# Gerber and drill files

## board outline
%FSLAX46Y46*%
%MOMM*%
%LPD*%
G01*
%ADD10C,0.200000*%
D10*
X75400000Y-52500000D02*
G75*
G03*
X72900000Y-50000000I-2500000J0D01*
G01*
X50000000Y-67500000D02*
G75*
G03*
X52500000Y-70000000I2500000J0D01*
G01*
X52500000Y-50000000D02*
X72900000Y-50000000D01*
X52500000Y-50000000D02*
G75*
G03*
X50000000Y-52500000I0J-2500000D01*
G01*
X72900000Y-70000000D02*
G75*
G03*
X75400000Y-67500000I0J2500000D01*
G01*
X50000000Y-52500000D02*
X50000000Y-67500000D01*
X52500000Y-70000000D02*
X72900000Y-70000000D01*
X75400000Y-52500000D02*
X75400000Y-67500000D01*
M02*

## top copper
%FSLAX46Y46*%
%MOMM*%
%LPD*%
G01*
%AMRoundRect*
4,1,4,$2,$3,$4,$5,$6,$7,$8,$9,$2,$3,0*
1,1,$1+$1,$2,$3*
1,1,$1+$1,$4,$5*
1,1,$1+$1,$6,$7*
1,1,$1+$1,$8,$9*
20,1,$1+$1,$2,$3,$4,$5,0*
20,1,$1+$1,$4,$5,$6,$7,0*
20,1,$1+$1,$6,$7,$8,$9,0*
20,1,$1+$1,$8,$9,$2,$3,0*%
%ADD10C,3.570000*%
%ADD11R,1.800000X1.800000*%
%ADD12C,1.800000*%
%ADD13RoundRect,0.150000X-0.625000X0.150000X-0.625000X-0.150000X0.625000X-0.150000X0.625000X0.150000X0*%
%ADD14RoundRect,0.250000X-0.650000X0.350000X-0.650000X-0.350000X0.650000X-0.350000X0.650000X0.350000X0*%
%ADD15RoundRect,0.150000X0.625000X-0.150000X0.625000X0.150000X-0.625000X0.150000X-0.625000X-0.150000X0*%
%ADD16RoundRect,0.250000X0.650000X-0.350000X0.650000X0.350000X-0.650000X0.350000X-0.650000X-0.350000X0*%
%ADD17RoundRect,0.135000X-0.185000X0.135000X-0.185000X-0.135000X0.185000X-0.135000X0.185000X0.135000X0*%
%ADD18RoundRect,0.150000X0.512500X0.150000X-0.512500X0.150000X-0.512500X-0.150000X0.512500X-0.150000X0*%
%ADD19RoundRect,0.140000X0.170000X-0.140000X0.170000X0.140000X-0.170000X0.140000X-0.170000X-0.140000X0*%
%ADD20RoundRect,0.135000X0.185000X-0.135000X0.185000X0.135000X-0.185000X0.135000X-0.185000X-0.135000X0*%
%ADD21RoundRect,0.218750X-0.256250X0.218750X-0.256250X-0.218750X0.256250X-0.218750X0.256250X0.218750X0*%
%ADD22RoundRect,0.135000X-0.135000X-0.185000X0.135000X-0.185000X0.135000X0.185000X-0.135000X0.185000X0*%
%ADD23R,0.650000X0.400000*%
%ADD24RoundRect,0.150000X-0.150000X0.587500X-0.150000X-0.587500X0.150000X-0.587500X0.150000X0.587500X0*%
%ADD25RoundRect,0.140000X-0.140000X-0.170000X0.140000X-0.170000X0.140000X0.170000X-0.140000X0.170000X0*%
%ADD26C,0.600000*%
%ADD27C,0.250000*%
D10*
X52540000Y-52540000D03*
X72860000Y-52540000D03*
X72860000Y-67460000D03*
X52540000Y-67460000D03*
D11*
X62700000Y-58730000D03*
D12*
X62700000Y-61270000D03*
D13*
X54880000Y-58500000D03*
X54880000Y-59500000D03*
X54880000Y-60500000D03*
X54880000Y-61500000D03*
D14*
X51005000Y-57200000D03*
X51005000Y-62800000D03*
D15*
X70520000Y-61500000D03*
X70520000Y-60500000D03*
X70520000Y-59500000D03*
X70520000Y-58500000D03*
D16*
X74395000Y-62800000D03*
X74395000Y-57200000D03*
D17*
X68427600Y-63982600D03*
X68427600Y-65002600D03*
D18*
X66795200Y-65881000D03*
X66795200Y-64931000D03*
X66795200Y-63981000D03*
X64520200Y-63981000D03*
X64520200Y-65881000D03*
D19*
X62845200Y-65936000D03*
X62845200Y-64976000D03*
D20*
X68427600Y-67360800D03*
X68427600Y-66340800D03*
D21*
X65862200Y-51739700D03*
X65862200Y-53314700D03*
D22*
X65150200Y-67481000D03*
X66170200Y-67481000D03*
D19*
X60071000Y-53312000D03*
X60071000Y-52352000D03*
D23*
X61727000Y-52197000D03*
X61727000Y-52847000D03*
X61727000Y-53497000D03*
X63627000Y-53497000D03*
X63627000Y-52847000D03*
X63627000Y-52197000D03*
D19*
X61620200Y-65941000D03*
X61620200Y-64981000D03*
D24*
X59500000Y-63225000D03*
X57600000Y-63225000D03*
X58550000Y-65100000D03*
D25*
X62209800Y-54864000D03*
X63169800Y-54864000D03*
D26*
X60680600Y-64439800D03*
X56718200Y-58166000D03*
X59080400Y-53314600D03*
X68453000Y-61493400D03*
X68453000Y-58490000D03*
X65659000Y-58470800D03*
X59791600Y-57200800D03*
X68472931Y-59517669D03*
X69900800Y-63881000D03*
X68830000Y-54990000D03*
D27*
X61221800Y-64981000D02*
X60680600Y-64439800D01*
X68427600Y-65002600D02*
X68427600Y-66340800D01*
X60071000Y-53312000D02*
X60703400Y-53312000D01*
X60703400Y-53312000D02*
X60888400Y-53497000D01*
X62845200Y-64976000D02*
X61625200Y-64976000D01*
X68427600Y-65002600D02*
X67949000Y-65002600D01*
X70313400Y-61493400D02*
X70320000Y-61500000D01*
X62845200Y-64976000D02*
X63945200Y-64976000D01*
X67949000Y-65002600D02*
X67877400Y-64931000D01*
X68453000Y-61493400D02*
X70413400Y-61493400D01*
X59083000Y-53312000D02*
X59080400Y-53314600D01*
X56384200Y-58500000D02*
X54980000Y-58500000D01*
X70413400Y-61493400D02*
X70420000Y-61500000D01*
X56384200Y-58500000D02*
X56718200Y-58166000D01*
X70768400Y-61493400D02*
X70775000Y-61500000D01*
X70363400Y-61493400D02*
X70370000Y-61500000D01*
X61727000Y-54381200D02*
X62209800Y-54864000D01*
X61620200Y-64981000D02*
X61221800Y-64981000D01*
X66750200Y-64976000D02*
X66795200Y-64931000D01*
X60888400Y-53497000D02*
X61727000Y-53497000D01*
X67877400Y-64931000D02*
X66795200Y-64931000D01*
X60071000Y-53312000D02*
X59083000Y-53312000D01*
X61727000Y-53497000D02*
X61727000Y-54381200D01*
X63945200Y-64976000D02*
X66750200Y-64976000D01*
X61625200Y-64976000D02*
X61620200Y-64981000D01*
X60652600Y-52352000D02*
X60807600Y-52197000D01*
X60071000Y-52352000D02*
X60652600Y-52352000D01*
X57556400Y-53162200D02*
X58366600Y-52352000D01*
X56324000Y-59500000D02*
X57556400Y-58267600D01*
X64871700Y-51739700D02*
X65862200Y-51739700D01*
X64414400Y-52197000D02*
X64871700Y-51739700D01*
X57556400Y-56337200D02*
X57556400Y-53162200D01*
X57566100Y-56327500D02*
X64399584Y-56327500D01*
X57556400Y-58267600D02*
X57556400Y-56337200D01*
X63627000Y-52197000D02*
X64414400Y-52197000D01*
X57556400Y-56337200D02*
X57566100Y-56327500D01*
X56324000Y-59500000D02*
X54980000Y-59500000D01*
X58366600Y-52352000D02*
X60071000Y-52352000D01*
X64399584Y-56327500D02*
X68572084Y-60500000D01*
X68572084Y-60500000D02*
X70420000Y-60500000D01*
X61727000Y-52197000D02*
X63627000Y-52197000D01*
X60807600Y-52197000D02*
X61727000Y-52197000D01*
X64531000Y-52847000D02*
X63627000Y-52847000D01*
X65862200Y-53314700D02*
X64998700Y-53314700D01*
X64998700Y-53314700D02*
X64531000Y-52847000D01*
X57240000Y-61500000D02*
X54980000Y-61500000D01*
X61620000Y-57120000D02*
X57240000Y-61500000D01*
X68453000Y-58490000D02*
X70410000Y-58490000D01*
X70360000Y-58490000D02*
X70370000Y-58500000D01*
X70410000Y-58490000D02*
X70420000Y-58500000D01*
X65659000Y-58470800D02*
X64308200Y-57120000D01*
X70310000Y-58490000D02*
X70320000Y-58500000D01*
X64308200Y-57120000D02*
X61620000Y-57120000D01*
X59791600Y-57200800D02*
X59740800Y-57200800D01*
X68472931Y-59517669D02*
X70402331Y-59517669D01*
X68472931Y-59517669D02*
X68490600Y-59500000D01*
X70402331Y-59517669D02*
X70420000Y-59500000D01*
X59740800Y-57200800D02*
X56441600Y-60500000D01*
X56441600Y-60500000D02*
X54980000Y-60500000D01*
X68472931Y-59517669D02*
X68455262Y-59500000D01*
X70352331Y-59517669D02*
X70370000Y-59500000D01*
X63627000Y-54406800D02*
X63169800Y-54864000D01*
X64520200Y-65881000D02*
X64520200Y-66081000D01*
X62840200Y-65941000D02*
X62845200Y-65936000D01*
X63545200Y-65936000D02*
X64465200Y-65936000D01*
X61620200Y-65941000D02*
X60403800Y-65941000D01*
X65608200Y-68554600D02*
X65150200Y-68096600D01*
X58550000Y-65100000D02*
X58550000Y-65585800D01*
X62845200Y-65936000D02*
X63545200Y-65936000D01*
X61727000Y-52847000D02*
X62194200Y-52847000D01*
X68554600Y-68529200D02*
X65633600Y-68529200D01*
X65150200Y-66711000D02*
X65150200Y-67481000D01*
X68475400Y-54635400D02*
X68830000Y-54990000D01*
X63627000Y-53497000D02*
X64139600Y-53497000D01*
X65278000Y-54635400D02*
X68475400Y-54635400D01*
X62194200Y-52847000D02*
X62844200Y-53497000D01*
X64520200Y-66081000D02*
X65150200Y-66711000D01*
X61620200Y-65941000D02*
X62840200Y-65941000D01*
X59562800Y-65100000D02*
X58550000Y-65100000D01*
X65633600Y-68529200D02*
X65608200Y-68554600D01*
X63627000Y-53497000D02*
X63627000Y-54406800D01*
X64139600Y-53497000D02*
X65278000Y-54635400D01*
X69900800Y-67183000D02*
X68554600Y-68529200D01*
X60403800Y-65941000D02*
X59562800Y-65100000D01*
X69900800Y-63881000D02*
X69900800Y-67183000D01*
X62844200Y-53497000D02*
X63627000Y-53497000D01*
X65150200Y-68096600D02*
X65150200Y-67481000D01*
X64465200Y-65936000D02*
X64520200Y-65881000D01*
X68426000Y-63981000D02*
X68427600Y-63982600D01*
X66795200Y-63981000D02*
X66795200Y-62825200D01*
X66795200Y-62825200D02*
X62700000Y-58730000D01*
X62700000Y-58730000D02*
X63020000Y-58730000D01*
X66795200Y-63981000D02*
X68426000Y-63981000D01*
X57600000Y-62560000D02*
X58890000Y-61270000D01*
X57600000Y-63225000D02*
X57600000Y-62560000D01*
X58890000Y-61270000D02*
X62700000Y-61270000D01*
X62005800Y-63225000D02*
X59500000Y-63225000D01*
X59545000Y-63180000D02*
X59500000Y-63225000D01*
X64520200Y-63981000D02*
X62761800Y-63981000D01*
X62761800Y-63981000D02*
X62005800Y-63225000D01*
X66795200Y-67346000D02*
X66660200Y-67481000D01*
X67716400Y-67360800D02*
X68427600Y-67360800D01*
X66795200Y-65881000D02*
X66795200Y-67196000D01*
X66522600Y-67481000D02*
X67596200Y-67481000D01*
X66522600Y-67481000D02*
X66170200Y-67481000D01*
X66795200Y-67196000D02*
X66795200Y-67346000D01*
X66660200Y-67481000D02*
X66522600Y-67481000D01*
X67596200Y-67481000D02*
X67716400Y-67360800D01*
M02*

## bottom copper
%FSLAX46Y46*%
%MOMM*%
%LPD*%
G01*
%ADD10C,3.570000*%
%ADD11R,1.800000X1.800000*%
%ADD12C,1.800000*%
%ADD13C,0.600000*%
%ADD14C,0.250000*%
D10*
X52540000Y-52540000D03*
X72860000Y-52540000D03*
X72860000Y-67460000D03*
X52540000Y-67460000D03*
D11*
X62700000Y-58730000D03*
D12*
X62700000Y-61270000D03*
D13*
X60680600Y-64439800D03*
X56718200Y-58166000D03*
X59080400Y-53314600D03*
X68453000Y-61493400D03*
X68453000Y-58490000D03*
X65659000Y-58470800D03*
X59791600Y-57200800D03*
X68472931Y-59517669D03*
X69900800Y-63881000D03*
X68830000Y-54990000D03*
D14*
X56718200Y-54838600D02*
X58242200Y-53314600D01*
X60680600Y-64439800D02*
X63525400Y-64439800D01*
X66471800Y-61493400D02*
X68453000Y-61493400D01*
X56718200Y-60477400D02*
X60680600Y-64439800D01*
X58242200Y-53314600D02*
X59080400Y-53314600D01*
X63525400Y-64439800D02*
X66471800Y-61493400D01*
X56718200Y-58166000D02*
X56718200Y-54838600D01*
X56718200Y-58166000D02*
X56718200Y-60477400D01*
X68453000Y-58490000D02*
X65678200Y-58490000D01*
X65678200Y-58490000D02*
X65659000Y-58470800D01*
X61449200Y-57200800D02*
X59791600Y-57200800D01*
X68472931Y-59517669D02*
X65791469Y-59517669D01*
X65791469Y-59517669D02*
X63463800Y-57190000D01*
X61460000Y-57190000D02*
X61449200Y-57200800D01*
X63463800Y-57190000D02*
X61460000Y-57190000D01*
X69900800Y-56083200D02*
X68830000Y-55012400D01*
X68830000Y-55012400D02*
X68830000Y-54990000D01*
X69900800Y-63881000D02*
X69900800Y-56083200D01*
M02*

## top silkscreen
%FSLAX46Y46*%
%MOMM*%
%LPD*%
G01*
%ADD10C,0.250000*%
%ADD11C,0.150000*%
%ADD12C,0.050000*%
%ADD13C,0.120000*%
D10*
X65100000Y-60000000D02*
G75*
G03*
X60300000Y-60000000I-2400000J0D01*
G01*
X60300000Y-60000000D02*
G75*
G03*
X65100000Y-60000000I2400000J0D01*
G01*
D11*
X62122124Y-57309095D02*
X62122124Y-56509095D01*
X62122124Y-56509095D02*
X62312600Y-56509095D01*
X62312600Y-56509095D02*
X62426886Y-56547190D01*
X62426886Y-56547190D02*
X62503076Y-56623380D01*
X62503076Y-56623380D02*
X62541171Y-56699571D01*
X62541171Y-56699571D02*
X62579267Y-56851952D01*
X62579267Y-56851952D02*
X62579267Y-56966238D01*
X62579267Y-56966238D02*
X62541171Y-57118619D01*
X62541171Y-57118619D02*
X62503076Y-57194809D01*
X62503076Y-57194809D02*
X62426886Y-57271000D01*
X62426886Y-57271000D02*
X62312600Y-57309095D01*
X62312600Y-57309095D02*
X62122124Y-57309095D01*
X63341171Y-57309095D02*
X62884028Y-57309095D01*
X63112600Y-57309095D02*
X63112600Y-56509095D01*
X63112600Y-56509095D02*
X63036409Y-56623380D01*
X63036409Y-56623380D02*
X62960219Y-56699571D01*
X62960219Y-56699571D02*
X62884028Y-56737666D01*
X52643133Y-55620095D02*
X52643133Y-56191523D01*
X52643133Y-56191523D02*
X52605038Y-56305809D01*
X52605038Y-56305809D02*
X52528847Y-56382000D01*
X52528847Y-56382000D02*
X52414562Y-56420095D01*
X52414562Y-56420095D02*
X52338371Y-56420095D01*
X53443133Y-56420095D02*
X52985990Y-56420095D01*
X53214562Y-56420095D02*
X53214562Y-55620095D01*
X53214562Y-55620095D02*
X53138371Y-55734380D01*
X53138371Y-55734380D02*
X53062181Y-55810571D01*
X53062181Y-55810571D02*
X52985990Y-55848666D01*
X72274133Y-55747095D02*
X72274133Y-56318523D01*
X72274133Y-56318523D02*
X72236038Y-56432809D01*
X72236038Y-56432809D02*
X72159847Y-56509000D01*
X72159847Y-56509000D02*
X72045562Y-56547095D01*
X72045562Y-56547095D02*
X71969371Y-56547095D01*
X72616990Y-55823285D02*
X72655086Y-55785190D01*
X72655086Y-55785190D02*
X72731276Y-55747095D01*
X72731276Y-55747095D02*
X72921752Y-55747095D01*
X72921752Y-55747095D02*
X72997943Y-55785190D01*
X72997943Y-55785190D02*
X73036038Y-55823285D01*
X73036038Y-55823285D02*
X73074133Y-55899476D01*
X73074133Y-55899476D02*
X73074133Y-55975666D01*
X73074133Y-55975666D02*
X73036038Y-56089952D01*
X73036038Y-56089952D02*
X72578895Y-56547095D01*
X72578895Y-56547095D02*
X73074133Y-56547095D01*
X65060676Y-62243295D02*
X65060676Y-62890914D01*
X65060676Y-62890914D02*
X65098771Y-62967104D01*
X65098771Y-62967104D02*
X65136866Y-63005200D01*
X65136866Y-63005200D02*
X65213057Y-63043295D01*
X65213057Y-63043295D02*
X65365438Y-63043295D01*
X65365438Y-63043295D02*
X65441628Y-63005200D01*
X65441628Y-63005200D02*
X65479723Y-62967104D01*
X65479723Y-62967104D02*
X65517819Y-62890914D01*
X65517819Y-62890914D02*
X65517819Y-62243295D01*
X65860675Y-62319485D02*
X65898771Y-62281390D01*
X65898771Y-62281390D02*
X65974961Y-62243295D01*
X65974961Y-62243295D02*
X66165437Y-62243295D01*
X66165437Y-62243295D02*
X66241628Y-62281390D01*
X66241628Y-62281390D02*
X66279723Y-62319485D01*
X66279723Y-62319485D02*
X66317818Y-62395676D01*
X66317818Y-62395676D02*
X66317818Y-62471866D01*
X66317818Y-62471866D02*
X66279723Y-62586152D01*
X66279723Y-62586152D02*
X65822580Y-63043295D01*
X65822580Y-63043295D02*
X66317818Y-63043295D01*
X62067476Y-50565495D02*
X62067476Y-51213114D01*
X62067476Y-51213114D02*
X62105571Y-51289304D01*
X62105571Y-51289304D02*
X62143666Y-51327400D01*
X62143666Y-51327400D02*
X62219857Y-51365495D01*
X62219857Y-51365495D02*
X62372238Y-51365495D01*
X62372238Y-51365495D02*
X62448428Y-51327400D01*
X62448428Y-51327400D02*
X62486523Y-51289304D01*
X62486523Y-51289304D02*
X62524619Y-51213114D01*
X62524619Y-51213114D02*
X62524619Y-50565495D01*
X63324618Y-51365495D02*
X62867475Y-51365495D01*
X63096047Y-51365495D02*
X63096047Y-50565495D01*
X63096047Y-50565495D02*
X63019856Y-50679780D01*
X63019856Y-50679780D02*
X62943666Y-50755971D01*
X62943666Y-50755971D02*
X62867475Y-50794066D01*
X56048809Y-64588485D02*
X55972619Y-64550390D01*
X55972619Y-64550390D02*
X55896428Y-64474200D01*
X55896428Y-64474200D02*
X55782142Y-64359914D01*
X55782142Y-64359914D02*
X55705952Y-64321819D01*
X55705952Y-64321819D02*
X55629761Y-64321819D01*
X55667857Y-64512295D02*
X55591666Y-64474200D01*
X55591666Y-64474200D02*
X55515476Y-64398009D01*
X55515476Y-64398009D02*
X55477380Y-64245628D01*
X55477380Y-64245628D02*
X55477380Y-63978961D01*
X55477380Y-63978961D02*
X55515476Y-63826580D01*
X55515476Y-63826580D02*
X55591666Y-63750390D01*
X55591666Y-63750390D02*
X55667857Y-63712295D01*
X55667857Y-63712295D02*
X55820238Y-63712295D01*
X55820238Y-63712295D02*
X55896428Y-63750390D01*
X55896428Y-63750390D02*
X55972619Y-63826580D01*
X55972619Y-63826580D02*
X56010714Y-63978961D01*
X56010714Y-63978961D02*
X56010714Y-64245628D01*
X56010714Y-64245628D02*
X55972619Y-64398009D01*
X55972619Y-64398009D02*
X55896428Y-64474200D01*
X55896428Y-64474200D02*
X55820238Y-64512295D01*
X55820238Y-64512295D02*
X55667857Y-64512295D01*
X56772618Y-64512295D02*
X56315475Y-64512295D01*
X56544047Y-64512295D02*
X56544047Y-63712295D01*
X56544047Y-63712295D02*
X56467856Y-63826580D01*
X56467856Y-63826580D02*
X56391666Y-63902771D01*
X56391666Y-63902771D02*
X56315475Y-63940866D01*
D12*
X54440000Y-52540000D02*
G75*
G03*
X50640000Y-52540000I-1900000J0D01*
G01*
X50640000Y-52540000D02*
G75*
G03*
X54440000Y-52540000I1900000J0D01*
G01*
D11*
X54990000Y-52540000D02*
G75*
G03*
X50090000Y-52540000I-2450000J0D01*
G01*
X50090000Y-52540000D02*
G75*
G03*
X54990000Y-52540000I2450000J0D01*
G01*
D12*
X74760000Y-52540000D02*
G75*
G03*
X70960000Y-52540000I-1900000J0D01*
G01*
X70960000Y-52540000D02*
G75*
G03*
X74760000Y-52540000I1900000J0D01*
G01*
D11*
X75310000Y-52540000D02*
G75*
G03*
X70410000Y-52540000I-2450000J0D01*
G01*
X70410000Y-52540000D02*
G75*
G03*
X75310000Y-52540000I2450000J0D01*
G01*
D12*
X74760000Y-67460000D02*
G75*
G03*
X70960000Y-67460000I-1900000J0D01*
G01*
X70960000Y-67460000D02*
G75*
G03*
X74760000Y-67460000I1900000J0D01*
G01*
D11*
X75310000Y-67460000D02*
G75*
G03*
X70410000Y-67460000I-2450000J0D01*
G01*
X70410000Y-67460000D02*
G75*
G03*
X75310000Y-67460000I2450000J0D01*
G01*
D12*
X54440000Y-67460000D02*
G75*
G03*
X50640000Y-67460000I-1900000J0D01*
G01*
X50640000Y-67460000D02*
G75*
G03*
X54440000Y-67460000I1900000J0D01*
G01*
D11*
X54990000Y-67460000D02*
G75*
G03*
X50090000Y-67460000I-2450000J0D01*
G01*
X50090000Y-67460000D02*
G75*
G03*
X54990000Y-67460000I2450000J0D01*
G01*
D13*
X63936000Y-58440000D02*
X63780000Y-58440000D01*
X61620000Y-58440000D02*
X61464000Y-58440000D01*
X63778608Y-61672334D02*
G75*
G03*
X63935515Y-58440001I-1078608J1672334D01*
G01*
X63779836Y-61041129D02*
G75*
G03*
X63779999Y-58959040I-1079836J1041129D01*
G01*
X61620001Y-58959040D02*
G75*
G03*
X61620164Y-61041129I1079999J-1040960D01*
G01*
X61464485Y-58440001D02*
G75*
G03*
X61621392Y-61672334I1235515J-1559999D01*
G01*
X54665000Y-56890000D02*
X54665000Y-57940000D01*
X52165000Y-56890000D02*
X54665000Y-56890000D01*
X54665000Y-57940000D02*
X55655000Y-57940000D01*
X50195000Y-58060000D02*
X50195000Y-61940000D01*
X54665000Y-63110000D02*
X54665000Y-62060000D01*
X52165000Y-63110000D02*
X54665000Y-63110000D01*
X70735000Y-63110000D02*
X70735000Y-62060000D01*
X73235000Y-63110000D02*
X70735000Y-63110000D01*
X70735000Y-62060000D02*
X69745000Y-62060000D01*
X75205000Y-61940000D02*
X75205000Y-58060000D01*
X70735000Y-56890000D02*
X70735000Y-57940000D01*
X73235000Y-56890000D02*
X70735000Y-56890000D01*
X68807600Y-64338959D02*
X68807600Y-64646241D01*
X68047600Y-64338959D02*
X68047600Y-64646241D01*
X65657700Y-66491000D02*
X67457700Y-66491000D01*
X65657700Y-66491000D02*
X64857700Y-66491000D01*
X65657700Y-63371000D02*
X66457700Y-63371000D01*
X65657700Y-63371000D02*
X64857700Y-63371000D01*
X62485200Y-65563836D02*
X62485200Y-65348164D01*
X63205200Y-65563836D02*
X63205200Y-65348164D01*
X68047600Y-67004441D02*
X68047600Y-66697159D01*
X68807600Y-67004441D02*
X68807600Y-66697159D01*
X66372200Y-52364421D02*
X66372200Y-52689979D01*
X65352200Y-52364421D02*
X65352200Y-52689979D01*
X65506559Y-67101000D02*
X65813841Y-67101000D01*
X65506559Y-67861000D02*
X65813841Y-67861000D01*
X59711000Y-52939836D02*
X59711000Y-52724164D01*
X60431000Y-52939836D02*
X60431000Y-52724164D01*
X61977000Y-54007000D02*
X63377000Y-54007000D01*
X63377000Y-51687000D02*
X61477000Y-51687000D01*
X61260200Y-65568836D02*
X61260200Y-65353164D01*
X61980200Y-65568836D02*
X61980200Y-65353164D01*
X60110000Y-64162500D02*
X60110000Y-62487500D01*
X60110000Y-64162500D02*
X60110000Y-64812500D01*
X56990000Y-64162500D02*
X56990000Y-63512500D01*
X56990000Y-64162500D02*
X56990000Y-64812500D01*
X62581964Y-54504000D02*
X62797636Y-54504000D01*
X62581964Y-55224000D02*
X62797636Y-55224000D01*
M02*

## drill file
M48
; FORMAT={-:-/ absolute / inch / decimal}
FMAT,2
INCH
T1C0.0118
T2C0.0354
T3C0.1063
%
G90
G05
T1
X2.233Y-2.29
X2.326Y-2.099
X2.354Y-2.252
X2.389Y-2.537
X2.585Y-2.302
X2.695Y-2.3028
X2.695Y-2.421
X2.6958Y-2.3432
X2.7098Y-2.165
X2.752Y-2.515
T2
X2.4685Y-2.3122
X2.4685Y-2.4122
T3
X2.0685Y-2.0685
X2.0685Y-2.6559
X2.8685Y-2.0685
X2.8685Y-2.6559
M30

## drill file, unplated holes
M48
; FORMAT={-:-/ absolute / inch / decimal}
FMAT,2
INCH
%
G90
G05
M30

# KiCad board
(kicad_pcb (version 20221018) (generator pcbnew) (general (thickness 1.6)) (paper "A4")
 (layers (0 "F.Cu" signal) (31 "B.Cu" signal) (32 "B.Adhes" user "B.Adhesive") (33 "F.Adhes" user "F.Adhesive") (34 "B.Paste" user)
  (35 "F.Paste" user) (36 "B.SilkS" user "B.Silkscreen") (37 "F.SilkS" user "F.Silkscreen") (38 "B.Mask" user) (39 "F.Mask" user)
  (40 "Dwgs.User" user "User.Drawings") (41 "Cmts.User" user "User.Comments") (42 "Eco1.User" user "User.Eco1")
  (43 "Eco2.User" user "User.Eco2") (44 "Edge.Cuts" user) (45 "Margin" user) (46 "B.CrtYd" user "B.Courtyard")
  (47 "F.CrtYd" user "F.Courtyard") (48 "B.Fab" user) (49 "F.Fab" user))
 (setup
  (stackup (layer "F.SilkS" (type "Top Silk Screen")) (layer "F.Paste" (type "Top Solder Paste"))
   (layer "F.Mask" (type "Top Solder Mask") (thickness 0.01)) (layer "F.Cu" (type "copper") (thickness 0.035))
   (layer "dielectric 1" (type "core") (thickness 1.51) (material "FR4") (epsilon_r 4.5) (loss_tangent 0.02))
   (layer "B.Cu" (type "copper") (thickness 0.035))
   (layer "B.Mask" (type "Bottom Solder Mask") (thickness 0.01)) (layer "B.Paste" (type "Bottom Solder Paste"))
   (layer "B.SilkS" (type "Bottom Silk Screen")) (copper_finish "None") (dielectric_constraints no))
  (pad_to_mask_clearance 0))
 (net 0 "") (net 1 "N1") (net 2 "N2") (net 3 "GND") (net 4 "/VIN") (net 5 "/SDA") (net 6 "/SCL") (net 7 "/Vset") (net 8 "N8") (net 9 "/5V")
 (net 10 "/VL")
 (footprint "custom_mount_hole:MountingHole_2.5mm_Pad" (layer "F.Cu") (at 52.54 52.54)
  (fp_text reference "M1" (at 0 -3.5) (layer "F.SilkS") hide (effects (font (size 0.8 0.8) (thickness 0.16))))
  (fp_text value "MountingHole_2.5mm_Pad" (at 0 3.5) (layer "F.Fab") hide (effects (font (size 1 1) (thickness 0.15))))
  (fp_circle (center 0 0) (end 1.9 0) (stroke (width 0.05) (type solid)) (fill none) (layer "F.SilkS"))
  (fp_circle (center 0 0) (end 2.45 0) (stroke (width 0.15) (type solid)) (fill none) (layer "F.SilkS"))
  (pad "~" thru_hole circle (at 0 0) (size 3.57 3.57) (drill 2.7) (layers "*.Cu" "*.Mask")))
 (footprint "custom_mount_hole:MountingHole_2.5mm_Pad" (layer "F.Cu") (at 72.86 52.54)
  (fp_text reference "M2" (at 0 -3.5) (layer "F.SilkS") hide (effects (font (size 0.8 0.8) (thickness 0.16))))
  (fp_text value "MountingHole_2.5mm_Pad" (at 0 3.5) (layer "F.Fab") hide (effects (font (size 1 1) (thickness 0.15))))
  (fp_circle (center 0 0) (end 1.9 0) (stroke (width 0.05) (type solid)) (fill none) (layer "F.SilkS"))
  (fp_circle (center 0 0) (end 2.45 0) (stroke (width 0.15) (type solid)) (fill none) (layer "F.SilkS"))
  (pad "~" thru_hole circle (at 0 0) (size 3.57 3.57) (drill 2.7) (layers "*.Cu" "*.Mask")))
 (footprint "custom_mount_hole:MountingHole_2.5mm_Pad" (layer "F.Cu") (at 72.86 67.46)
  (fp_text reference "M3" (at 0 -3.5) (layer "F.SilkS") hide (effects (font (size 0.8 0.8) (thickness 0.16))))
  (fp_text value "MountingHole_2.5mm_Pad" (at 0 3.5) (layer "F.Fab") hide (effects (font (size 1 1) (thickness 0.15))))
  (fp_circle (center 0 0) (end 1.9 0) (stroke (width 0.05) (type solid)) (fill none) (layer "F.SilkS"))
  (fp_circle (center 0 0) (end 2.45 0) (stroke (width 0.15) (type solid)) (fill none) (layer "F.SilkS"))
  (pad "~" thru_hole circle (at 0 0) (size 3.57 3.57) (drill 2.7) (layers "*.Cu" "*.Mask")))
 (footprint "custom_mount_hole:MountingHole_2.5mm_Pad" (layer "F.Cu") (at 52.54 67.46)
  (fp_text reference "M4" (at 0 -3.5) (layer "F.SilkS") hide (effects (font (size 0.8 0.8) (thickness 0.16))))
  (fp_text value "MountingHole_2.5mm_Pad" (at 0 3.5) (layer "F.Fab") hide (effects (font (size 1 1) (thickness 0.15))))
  (fp_circle (center 0 0) (end 1.9 0) (stroke (width 0.05) (type solid)) (fill none) (layer "F.SilkS"))
  (fp_circle (center 0 0) (end 2.45 0) (stroke (width 0.15) (type solid)) (fill none) (layer "F.SilkS"))
  (pad "~" thru_hole circle (at 0 0) (size 3.57 3.57) (drill 2.7) (layers "*.Cu" "*.Mask")))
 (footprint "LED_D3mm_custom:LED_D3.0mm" (layer "F.Cu") (at 62.7 58.73 -90)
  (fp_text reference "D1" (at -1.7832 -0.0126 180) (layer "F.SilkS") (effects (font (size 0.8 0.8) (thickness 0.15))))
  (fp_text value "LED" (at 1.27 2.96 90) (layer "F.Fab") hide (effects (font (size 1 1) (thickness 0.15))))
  (fp_line (start -0.29 -1.236) (end -0.29 -1.08) (stroke (width 0.12) (type solid)) (layer "F.SilkS"))
  (fp_line (start -0.29 1.08) (end -0.29 1.236) (stroke (width 0.12) (type solid)) (layer "F.SilkS"))
  (fp_arc (start -0.29 -1.235516) (mid 1.366487 -1.987659) (end 2.942335 -1.078608) (stroke (width 0.12) (type solid)) (layer "F.SilkS"))
  (fp_arc (start 0.229039 -1.08) (mid 1.270117 -1.5) (end 2.31113 -1.079837) (stroke (width 0.12) (type solid)) (layer "F.SilkS"))
  (fp_arc (start 2.31113 1.079837) (mid 1.270117 1.5) (end 0.229039 1.08) (stroke (width 0.12) (type solid)) (layer "F.SilkS"))
  (fp_arc (start 2.942335 1.078608) (mid 1.366487 1.987659) (end -0.29 1.235516) (stroke (width 0.12) (type solid)) (layer "F.SilkS"))
  (pad "1" thru_hole rect (at 0 0 270) (size 1.8 1.8) (drill 0.9) (layers "*.Cu" "*.Mask") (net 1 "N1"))
  (pad "2" thru_hole circle (at 2.54 0 270) (size 1.8 1.8) (drill 0.9) (layers "*.Cu" "*.Mask") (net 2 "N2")))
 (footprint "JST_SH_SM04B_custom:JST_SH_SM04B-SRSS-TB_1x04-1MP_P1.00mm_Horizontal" (layer "F.Cu") (at 52.88 60 -90)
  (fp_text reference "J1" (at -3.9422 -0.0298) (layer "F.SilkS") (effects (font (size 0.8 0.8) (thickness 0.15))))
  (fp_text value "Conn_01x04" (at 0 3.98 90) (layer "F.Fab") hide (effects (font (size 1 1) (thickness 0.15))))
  (fp_line (start -3.11 -1.785) (end -2.06 -1.785) (stroke (width 0.12) (type solid)) (layer "F.SilkS"))
  (fp_line (start -3.11 0.715) (end -3.11 -1.785) (stroke (width 0.12) (type solid)) (layer "F.SilkS"))
  (fp_line (start -2.06 -1.785) (end -2.06 -2.775) (stroke (width 0.12) (type solid)) (layer "F.SilkS"))
  (fp_line (start -1.94 2.685) (end 1.94 2.685) (stroke (width 0.12) (type solid)) (layer "F.SilkS"))
  (fp_line (start 3.11 -1.785) (end 2.06 -1.785) (stroke (width 0.12) (type solid)) (layer "F.SilkS"))
  (fp_line (start 3.11 0.715) (end 3.11 -1.785) (stroke (width 0.12) (type solid)) (layer "F.SilkS"))
  (pad "1" smd roundrect (at -1.5 -2 270) (size 0.6 1.55) (layers "F.Cu" "F.Paste" "F.Mask") (roundrect_rratio 0.25) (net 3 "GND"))
  (pad "2" smd roundrect (at -0.5 -2 270) (size 0.6 1.55) (layers "F.Cu" "F.Paste" "F.Mask") (roundrect_rratio 0.25) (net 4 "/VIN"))
  (pad "3" smd roundrect (at 0.5 -2 270) (size 0.6 1.55) (layers "F.Cu" "F.Paste" "F.Mask") (roundrect_rratio 0.25) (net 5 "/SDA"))
  (pad "4" smd roundrect (at 1.5 -2 270) (size 0.6 1.55) (layers "F.Cu" "F.Paste" "F.Mask") (roundrect_rratio 0.25) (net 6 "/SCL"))
  (pad "MP" smd roundrect (at -2.8 1.875 270) (size 1.2 1.8) (layers "F.Cu" "F.Paste" "F.Mask") (roundrect_rratio 0.2083333333))
  (pad "MP" smd roundrect (at 2.8 1.875 270) (size 1.2 1.8) (layers "F.Cu" "F.Paste" "F.Mask") (roundrect_rratio 0.2083333333)))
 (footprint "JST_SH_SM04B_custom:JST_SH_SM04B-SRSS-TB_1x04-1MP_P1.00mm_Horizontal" (layer "F.Cu") (at 72.52 60 90)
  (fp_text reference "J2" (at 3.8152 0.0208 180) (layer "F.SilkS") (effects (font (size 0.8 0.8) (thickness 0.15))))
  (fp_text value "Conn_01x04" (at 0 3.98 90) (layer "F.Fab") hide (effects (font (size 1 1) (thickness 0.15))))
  (fp_line (start -3.11 -1.785) (end -2.06 -1.785) (stroke (width 0.12) (type solid)) (layer "F.SilkS"))
  (fp_line (start -3.11 0.715) (end -3.11 -1.785) (stroke (width 0.12) (type solid)) (layer "F.SilkS"))
  (fp_line (start -2.06 -1.785) (end -2.06 -2.775) (stroke (width 0.12) (type solid)) (layer "F.SilkS"))
  (fp_line (start -1.94 2.685) (end 1.94 2.685) (stroke (width 0.12) (type solid)) (layer "F.SilkS"))
  (fp_line (start 3.11 -1.785) (end 2.06 -1.785) (stroke (width 0.12) (type solid)) (layer "F.SilkS"))
  (fp_line (start 3.11 0.715) (end 3.11 -1.785) (stroke (width 0.12) (type solid)) (layer "F.SilkS"))
  (pad "1" smd roundrect (at -1.5 -2 90) (size 0.6 1.55) (layers "F.Cu" "F.Paste" "F.Mask") (roundrect_rratio 0.25) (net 3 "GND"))
  (pad "2" smd roundrect (at -0.5 -2 90) (size 0.6 1.55) (layers "F.Cu" "F.Paste" "F.Mask") (roundrect_rratio 0.25) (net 4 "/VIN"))
  (pad "3" smd roundrect (at 0.5 -2 90) (size 0.6 1.55) (layers "F.Cu" "F.Paste" "F.Mask") (roundrect_rratio 0.25) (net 5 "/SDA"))
  (pad "4" smd roundrect (at 1.5 -2 90) (size 0.6 1.55) (layers "F.Cu" "F.Paste" "F.Mask") (roundrect_rratio 0.25) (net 6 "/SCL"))
  (pad "MP" smd roundrect (at -2.8 1.875 90) (size 1.2 1.8) (layers "F.Cu" "F.Paste" "F.Mask") (roundrect_rratio 0.2083333333))
  (pad "MP" smd roundrect (at 2.8 1.875 90) (size 1.2 1.8) (layers "F.Cu" "F.Paste" "F.Mask") (roundrect_rratio 0.2083333333)))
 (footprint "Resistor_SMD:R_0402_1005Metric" (layer "F.Cu") (at 68.4276 64.4926 -90)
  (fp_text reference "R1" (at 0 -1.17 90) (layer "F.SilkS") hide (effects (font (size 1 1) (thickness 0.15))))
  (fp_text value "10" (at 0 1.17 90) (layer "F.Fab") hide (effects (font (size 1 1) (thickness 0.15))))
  (fp_line (start -0.153641 -0.38) (end 0.153641 -0.38) (stroke (width 0.12) (type solid)) (layer "F.SilkS"))
  (fp_line (start -0.153641 0.38) (end 0.153641 0.38) (stroke (width 0.12) (type solid)) (layer "F.SilkS"))
  (pad "1" smd roundrect (at -0.51 0 270) (size 0.54 0.64) (layers "F.Cu" "F.Paste" "F.Mask") (roundrect_rratio 0.25) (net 1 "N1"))
  (pad "2" smd roundrect (at 0.51 0 270) (size 0.54 0.64) (layers "F.Cu" "F.Paste" "F.Mask") (roundrect_rratio 0.25) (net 3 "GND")))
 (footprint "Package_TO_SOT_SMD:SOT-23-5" (layer "F.Cu") (at 65.6577 64.931 180)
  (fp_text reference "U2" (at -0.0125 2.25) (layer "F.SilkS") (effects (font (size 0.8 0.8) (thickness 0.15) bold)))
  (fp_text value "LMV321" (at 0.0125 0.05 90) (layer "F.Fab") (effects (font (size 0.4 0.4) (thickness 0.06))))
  (fp_line (start 0 -1.56) (end -1.8 -1.56) (stroke (width 0.12) (type solid)) (layer "F.SilkS"))
  (fp_line (start 0 -1.56) (end 0.8 -1.56) (stroke (width 0.12) (type solid)) (layer "F.SilkS"))
  (fp_line (start 0 1.56) (end -0.8 1.56) (stroke (width 0.12) (type solid)) (layer "F.SilkS"))
  (fp_line (start 0 1.56) (end 0.8 1.56) (stroke (width 0.12) (type solid)) (layer "F.SilkS"))
  (pad "1" smd roundrect (at -1.1375 -0.95 180) (size 1.325 0.6) (layers "F.Cu" "F.Paste" "F.Mask") (roundrect_rratio 0.25) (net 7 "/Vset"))
  (pad "2" smd roundrect (at -1.1375 0 180) (size 1.325 0.6) (layers "F.Cu" "F.Paste" "F.Mask") (roundrect_rratio 0.25) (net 3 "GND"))
  (pad "3" smd roundrect (at -1.1375 0.95 180) (size 1.325 0.6) (layers "F.Cu" "F.Paste" "F.Mask") (roundrect_rratio 0.25) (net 1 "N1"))
  (pad "4" smd roundrect (at 1.1375 0.95 180) (size 1.325 0.6) (layers "F.Cu" "F.Paste" "F.Mask") (roundrect_rratio 0.25) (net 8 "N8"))
  (pad "5" smd roundrect (at 1.1375 -0.95 180) (size 1.325 0.6) (layers "F.Cu" "F.Paste" "F.Mask") (roundrect_rratio 0.25) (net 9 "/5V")))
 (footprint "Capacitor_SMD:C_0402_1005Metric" (layer "F.Cu") (at 62.8452 65.456 90)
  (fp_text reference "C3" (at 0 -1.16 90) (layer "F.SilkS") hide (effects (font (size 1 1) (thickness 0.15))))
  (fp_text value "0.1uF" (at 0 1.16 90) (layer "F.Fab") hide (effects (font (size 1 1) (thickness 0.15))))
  (fp_line (start -0.107836 -0.36) (end 0.107836 -0.36) (stroke (width 0.12) (type solid)) (layer "F.SilkS"))
  (fp_line (start -0.107836 0.36) (end 0.107836 0.36) (stroke (width 0.12) (type solid)) (layer "F.SilkS"))
  (pad "1" smd roundrect (at -0.48 0 90) (size 0.56 0.62) (layers "F.Cu" "F.Paste" "F.Mask") (roundrect_rratio 0.25) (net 9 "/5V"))
  (pad "2" smd roundrect (at 0.48 0 90) (size 0.56 0.62) (layers "F.Cu" "F.Paste" "F.Mask") (roundrect_rratio 0.25) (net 3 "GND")))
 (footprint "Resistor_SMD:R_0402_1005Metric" (layer "F.Cu") (at 68.4276 66.8508 90)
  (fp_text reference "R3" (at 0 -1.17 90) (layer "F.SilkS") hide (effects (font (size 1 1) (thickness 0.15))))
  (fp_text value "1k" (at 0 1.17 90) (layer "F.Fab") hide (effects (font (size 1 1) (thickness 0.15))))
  (fp_line (start -0.153641 -0.38) (end 0.153641 -0.38) (stroke (width 0.12) (type solid)) (layer "F.SilkS"))
  (fp_line (start -0.153641 0.38) (end 0.153641 0.38) (stroke (width 0.12) (type solid)) (layer "F.SilkS"))
  (pad "1" smd roundrect (at -0.51 0 90) (size 0.54 0.64) (layers "F.Cu" "F.Paste" "F.Mask") (roundrect_rratio 0.25) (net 7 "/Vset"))
  (pad "2" smd roundrect (at 0.51 0 90) (size 0.54 0.64) (layers "F.Cu" "F.Paste" "F.Mask") (roundrect_rratio 0.25) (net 3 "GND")))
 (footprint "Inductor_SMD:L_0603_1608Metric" (layer "F.Cu") (at 65.8622 52.5272 -90)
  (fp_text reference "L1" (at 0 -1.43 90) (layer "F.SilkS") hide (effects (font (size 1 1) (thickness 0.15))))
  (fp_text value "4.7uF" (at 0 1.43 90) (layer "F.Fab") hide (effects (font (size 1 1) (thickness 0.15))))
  (fp_line (start -0.162779 -0.51) (end 0.162779 -0.51) (stroke (width 0.12) (type solid)) (layer "F.SilkS"))
  (fp_line (start -0.162779 0.51) (end 0.162779 0.51) (stroke (width 0.12) (type solid)) (layer "F.SilkS"))
  (pad "1" smd roundrect (at -0.7875 0 270) (size 0.875 0.95) (layers "F.Cu" "F.Paste" "F.Mask") (roundrect_rratio 0.25) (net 4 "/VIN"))
  (pad "2" smd roundrect (at 0.7875 0 270) (size 0.875 0.95) (layers "F.Cu" "F.Paste" "F.Mask") (roundrect_rratio 0.25) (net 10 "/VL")))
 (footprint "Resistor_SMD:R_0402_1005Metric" (layer "F.Cu") (at 65.6602 67.481)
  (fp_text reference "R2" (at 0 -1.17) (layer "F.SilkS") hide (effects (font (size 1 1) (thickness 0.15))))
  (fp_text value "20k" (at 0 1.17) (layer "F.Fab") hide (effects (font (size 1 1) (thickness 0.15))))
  (fp_line (start -0.153641 -0.38) (end 0.153641 -0.38) (stroke (width 0.12) (type solid)) (layer "F.SilkS"))
  (fp_line (start -0.153641 0.38) (end 0.153641 0.38) (stroke (width 0.12) (type solid)) (layer "F.SilkS"))
  (pad "1" smd roundrect (at -0.51 0) (size 0.54 0.64) (layers "F.Cu" "F.Paste" "F.Mask") (roundrect_rratio 0.25) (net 9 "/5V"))
  (pad "2" smd roundrect (at 0.51 0) (size 0.54 0.64) (layers "F.Cu" "F.Paste" "F.Mask") (roundrect_rratio 0.25) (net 7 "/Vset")))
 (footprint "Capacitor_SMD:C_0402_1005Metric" (layer "F.Cu") (at 60.071 52.832 90)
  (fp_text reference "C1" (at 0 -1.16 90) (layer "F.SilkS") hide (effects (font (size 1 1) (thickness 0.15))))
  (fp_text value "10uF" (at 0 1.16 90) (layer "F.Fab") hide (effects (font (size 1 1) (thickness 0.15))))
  (fp_line (start -0.107836 -0.36) (end 0.107836 -0.36) (stroke (width 0.12) (type solid)) (layer "F.SilkS"))
  (fp_line (start -0.107836 0.36) (end 0.107836 0.36) (stroke (width 0.12) (type solid)) (layer "F.SilkS"))
  (pad "1" smd roundrect (at -0.48 0 90) (size 0.56 0.62) (layers "F.Cu" "F.Paste" "F.Mask") (roundrect_rratio 0.25) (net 3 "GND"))
  (pad "2" smd roundrect (at 0.48 0 90) (size 0.56 0.62) (layers "F.Cu" "F.Paste" "F.Mask") (roundrect_rratio 0.25) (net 4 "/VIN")))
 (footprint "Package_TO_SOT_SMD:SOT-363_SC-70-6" (layer "F.Cu") (at 62.677 52.847)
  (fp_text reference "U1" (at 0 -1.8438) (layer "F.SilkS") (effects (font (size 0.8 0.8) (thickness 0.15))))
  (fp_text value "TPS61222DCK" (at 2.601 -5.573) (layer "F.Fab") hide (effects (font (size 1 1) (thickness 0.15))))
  (fp_line (start -0.7 1.16) (end 0.7 1.16) (stroke (width 0.12) (type solid)) (layer "F.SilkS"))
  (fp_line (start 0.7 -1.16) (end -1.2 -1.16) (stroke (width 0.12) (type solid)) (layer "F.SilkS"))
  (pad "1" smd rect (at -0.95 -0.65) (size 0.65 0.4) (layers "F.Cu" "F.Paste" "F.Mask") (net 4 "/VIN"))
  (pad "2" smd rect (at -0.95 0) (size 0.65 0.4) (layers "F.Cu" "F.Paste" "F.Mask") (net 9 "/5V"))
  (pad "3" smd rect (at -0.95 0.65) (size 0.65 0.4) (layers "F.Cu" "F.Paste" "F.Mask") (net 3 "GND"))
  (pad "4" smd rect (at 0.95 0.65) (size 0.65 0.4) (layers "F.Cu" "F.Paste" "F.Mask") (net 9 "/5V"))
  (pad "5" smd rect (at 0.95 0) (size 0.65 0.4) (layers "F.Cu" "F.Paste" "F.Mask") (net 10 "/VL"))
  (pad "6" smd rect (at 0.95 -0.65) (size 0.65 0.4) (layers "F.Cu" "F.Paste" "F.Mask") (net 4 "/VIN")))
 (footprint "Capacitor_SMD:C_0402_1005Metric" (layer "F.Cu") (at 61.6202 65.461 90)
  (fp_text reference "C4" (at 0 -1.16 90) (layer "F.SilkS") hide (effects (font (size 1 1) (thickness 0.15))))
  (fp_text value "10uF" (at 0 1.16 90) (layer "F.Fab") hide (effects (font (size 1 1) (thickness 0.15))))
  (fp_line (start -0.107836 -0.36) (end 0.107836 -0.36) (stroke (width 0.12) (type solid)) (layer "F.SilkS"))
  (fp_line (start -0.107836 0.36) (end 0.107836 0.36) (stroke (width 0.12) (type solid)) (layer "F.SilkS"))
  (pad "1" smd roundrect (at -0.48 0 90) (size 0.56 0.62) (layers "F.Cu" "F.Paste" "F.Mask") (roundrect_rratio 0.25) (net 9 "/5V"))
  (pad "2" smd roundrect (at 0.48 0 90) (size 0.56 0.62) (layers "F.Cu" "F.Paste" "F.Mask") (roundrect_rratio 0.25) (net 3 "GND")))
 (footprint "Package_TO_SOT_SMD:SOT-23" (layer "F.Cu") (at 58.55 64.1625 -90)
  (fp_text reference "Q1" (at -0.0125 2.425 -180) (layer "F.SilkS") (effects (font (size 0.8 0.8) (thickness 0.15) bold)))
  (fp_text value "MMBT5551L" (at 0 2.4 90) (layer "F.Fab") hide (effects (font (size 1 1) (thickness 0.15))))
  (fp_line (start 0 -1.56) (end -1.675 -1.56) (stroke (width 0.12) (type solid)) (layer "F.SilkS"))
  (fp_line (start 0 -1.56) (end 0.65 -1.56) (stroke (width 0.12) (type solid)) (layer "F.SilkS"))
  (fp_line (start 0 1.56) (end -0.65 1.56) (stroke (width 0.12) (type solid)) (layer "F.SilkS"))
  (fp_line (start 0 1.56) (end 0.65 1.56) (stroke (width 0.12) (type solid)) (layer "F.SilkS"))
  (pad "1" smd roundrect (at -0.9375 -0.95 270) (size 1.475 0.6) (layers "F.Cu" "F.Paste" "F.Mask") (roundrect_rratio 0.25) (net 8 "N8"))
  (pad "2" smd roundrect (at -0.9375 0.95 270) (size 1.475 0.6) (layers "F.Cu" "F.Paste" "F.Mask") (roundrect_rratio 0.25) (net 2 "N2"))
  (pad "3" smd roundrect (at 0.9375 0 270) (size 1.475 0.6) (layers "F.Cu" "F.Paste" "F.Mask") (roundrect_rratio 0.25) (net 9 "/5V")))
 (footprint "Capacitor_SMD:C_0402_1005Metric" (layer "F.Cu") (at 62.6898 54.864)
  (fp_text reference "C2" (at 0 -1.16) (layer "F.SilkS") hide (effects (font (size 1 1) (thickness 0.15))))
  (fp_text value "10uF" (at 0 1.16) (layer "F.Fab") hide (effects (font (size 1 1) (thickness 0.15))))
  (fp_line (start -0.107836 -0.36) (end 0.107836 -0.36) (stroke (width 0.12) (type solid)) (layer "F.SilkS"))
  (fp_line (start -0.107836 0.36) (end 0.107836 0.36) (stroke (width 0.12) (type solid)) (layer "F.SilkS"))
  (pad "1" smd roundrect (at -0.48 0) (size 0.56 0.62) (layers "F.Cu" "F.Paste" "F.Mask") (roundrect_rratio 0.25) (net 3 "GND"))
  (pad "2" smd roundrect (at 0.48 0) (size 0.56 0.62) (layers "F.Cu" "F.Paste" "F.Mask") (roundrect_rratio 0.25) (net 9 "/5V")))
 (gr_circle (center 62.7 60) (end 65.1 60) (stroke (width 0.25) (type solid)) (fill none) (layer "F.SilkS"))
 (gr_arc (start 72.9 50) (mid 74.667767 50.732233) (end 75.4 52.5) (stroke (width 0.2) (type solid)) (layer "Edge.Cuts"))
 (gr_arc (start 52.5 70) (mid 50.732233 69.267767) (end 50 67.5) (stroke (width 0.2) (type solid)) (layer "Edge.Cuts"))
 (gr_line (start 52.5 50) (end 72.9 50) (stroke (width 0.2) (type solid)) (layer "Edge.Cuts"))
 (gr_arc (start 50 52.5) (mid 50.732233 50.732233) (end 52.5 50) (stroke (width 0.2) (type solid)) (layer "Edge.Cuts"))
 (gr_arc (start 75.4 67.5) (mid 74.667767 69.267767) (end 72.9 70) (stroke (width 0.2) (type solid)) (layer "Edge.Cuts"))
 (gr_line (start 50 52.5) (end 50 67.5) (stroke (width 0.2) (type solid)) (layer "Edge.Cuts"))
 (gr_line (start 52.5 70) (end 72.9 70) (stroke (width 0.2) (type solid)) (layer "Edge.Cuts"))
 (gr_line (start 75.4 52.5) (end 75.4 67.5) (stroke (width 0.2) (type solid)) (layer "Edge.Cuts"))
 (segment (start 61.2218 64.981) (end 60.6806 64.4398) (width 0.25) (layer "F.Cu") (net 3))
 (segment (start 68.4276 65.0026) (end 68.4276 66.3408) (width 0.25) (layer "F.Cu") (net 3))
 (segment (start 60.071 53.312) (end 60.7034 53.312) (width 0.25) (layer "F.Cu") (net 3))
 (segment (start 60.7034 53.312) (end 60.8884 53.497) (width 0.25) (layer "F.Cu") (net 3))
 (segment (start 62.8452 64.976) (end 61.6252 64.976) (width 0.25) (layer "F.Cu") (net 3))
 (segment (start 68.4276 65.0026) (end 67.949 65.0026) (width 0.25) (layer "F.Cu") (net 3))
 (segment (start 70.3134 61.4934) (end 70.32 61.5) (width 0.25) (layer "F.Cu") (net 3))
 (segment (start 62.8452 64.976) (end 63.9452 64.976) (width 0.25) (layer "F.Cu") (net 3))
 (segment (start 67.949 65.0026) (end 67.8774 64.931) (width 0.25) (layer "F.Cu") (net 3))
 (segment (start 68.453 61.4934) (end 70.4134 61.4934) (width 0.25) (layer "F.Cu") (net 3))
 (segment (start 59.083 53.312) (end 59.0804 53.3146) (width 0.25) (layer "F.Cu") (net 3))
 (segment (start 56.3842 58.5) (end 54.98 58.5) (width 0.25) (layer "F.Cu") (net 3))
 (segment (start 70.4134 61.4934) (end 70.42 61.5) (width 0.25) (layer "F.Cu") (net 3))
 (segment (start 56.3842 58.5) (end 56.7182 58.166) (width 0.25) (layer "F.Cu") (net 3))
 (segment (start 70.7684 61.4934) (end 70.775 61.5) (width 0.25) (layer "F.Cu") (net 3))
 (segment (start 70.3634 61.4934) (end 70.37 61.5) (width 0.25) (layer "F.Cu") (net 3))
 (segment (start 61.727 54.3812) (end 62.2098 54.864) (width 0.25) (layer "F.Cu") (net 3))
 (segment (start 61.6202 64.981) (end 61.2218 64.981) (width 0.25) (layer "F.Cu") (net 3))
 (segment (start 66.7502 64.976) (end 66.7952 64.931) (width 0.25) (layer "F.Cu") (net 3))
 (segment (start 60.8884 53.497) (end 61.727 53.497) (width 0.25) (layer "F.Cu") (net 3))
 (segment (start 67.8774 64.931) (end 66.7952 64.931) (width 0.25) (layer "F.Cu") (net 3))
 (segment (start 60.071 53.312) (end 59.083 53.312) (width 0.25) (layer "F.Cu") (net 3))
 (segment (start 61.727 53.497) (end 61.727 54.3812) (width 0.25) (layer "F.Cu") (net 3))
 (segment (start 63.9452 64.976) (end 66.7502 64.976) (width 0.25) (layer "F.Cu") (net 3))
 (segment (start 61.6252 64.976) (end 61.6202 64.981) (width 0.25) (layer "F.Cu") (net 3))
 (via (at 60.6806 64.4398) (size 0.6) (drill 0.3) (layers "F.Cu" "B.Cu") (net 3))
 (via (at 56.7182 58.166) (size 0.6) (drill 0.3) (layers "F.Cu" "B.Cu") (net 3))
 (via (at 59.0804 53.3146) (size 0.6) (drill 0.3) (layers "F.Cu" "B.Cu") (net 3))
 (via (at 68.453 61.4934) (size 0.6) (drill 0.3) (layers "F.Cu" "B.Cu") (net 3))
 (segment (start 56.7182 54.8386) (end 58.2422 53.3146) (width 0.25) (layer "B.Cu") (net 3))
 (segment (start 60.6806 64.4398) (end 63.5254 64.4398) (width 0.25) (layer "B.Cu") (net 3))
 (segment (start 66.4718 61.4934) (end 68.453 61.4934) (width 0.25) (layer "B.Cu") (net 3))
 (segment (start 56.7182 60.4774) (end 60.6806 64.4398) (width 0.25) (layer "B.Cu") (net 3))
 (segment (start 58.2422 53.3146) (end 59.0804 53.3146) (width 0.25) (layer "B.Cu") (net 3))
 (segment (start 63.5254 64.4398) (end 66.4718 61.4934) (width 0.25) (layer "B.Cu") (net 3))
 (segment (start 56.7182 58.166) (end 56.7182 54.8386) (width 0.25) (layer "B.Cu") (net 3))
 (segment (start 56.7182 58.166) (end 56.7182 60.4774) (width 0.25) (layer "B.Cu") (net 3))
 (segment (start 60.6526 52.352) (end 60.8076 52.197) (width 0.25) (layer "F.Cu") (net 4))
 (segment (start 60.071 52.352) (end 60.6526 52.352) (width 0.25) (layer "F.Cu") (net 4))
 (segment (start 57.5564 53.1622) (end 58.3666 52.352) (width 0.25) (layer "F.Cu") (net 4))
 (segment (start 56.324 59.5) (end 57.5564 58.2676) (width 0.25) (layer "F.Cu") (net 4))
 (segment (start 64.8717 51.7397) (end 65.8622 51.7397) (width 0.25) (layer "F.Cu") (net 4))
 (segment (start 64.4144 52.197) (end 64.8717 51.7397) (width 0.25) (layer "F.Cu") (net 4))
 (segment (start 57.5564 56.3372) (end 57.5564 53.1622) (width 0.25) (layer "F.Cu") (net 4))
 (segment (start 57.5661 56.3275) (end 64.399584 56.3275) (width 0.25) (layer "F.Cu") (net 4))
 (segment (start 57.5564 58.2676) (end 57.5564 56.3372) (width 0.25) (layer "F.Cu") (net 4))
 (segment (start 63.627 52.197) (end 64.4144 52.197) (width 0.25) (layer "F.Cu") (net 4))
 (segment (start 57.5564 56.3372) (end 57.5661 56.3275) (width 0.25) (layer "F.Cu") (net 4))
 (segment (start 56.324 59.5) (end 54.98 59.5) (width 0.25) (layer "F.Cu") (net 4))
 (segment (start 58.3666 52.352) (end 60.071 52.352) (width 0.25) (layer "F.Cu") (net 4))
 (segment (start 64.399584 56.3275) (end 68.572084 60.5) (width 0.25) (layer "F.Cu") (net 4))
 (segment (start 68.572084 60.5) (end 70.42 60.5) (width 0.25) (layer "F.Cu") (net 4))
 (segment (start 61.727 52.197) (end 63.627 52.197) (width 0.25) (layer "F.Cu") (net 4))
 (segment (start 60.8076 52.197) (end 61.727 52.197) (width 0.25) (layer "F.Cu") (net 4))
 (segment (start 64.531 52.847) (end 63.627 52.847) (width 0.25) (layer "F.Cu") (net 10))
 (segment (start 65.8622 53.3147) (end 64.9987 53.3147) (width 0.25) (layer "F.Cu") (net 10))
 (segment (start 64.9987 53.3147) (end 64.531 52.847) (width 0.25) (layer "F.Cu") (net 10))
 (segment (start 57.24 61.5) (end 54.98 61.5) (width 0.25) (layer "F.Cu") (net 6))
 (segment (start 61.62 57.12) (end 57.24 61.5) (width 0.25) (layer "F.Cu") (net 6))
 (segment (start 68.453 58.49) (end 70.41 58.49) (width 0.25) (layer "F.Cu") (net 6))
 (segment (start 70.36 58.49) (end 70.37 58.5) (width 0.25) (layer "F.Cu") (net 6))
 (segment (start 70.41 58.49) (end 70.42 58.5) (width 0.25) (layer "F.Cu") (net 6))
 (segment (start 65.659 58.4708) (end 64.3082 57.12) (width 0.25) (layer "F.Cu") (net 6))
 (segment (start 70.31 58.49) (end 70.32 58.5) (width 0.25) (layer "F.Cu") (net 6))
 (segment (start 64.3082 57.12) (end 61.62 57.12) (width 0.25) (layer "F.Cu") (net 6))
 (via (at 68.453 58.49) (size 0.6) (drill 0.3) (layers "F.Cu" "B.Cu") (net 6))
 (via (at 65.659 58.4708) (size 0.6) (drill 0.3) (layers "F.Cu" "B.Cu") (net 6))
 (segment (start 68.453 58.49) (end 65.6782 58.49) (width 0.25) (layer "B.Cu") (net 6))
 (segment (start 65.6782 58.49) (end 65.659 58.4708) (width 0.25) (layer "B.Cu") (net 6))
 (segment (start 59.7916 57.2008) (end 59.7408 57.2008) (width 0.25) (layer "F.Cu") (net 5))
 (segment (start 68.472931 59.517669) (end 70.402331 59.517669) (width 0.25) (layer "F.Cu") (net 5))
 (segment (start 68.472931 59.517669) (end 68.4906 59.5) (width 0.25) (layer "F.Cu") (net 5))
 (segment (start 70.402331 59.517669) (end 70.42 59.5) (width 0.25) (layer "F.Cu") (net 5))
 (segment (start 59.7408 57.2008) (end 56.4416 60.5) (width 0.25) (layer "F.Cu") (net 5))
 (segment (start 56.4416 60.5) (end 54.98 60.5) (width 0.25) (layer "F.Cu") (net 5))
 (segment (start 68.472931 59.517669) (end 68.455262 59.5) (width 0.25) (layer "F.Cu") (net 5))
 (segment (start 70.352331 59.517669) (end 70.37 59.5) (width 0.25) (layer "F.Cu") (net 5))
 (via (at 59.7916 57.2008) (size 0.6) (drill 0.3) (layers "F.Cu" "B.Cu") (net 5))
 (via (at 68.472931 59.517669) (size 0.6) (drill 0.3) (layers "F.Cu" "B.Cu") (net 5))
 (segment (start 61.4492 57.2008) (end 59.7916 57.2008) (width 0.25) (layer "B.Cu") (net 5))
 (segment (start 68.472931 59.517669) (end 65.791469 59.517669) (width 0.25) (layer "B.Cu") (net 5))
 (segment (start 65.791469 59.517669) (end 63.4638 57.19) (width 0.25) (layer "B.Cu") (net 5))
 (segment (start 61.46 57.19) (end 61.4492 57.2008) (width 0.25) (layer "B.Cu") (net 5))
 (segment (start 63.4638 57.19) (end 61.46 57.19) (width 0.25) (layer "B.Cu") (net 5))
 (segment (start 63.627 54.4068) (end 63.1698 54.864) (width 0.25) (layer "F.Cu") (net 9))
 (segment (start 64.5202 65.881) (end 64.5202 66.081) (width 0.25) (layer "F.Cu") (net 9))
 (segment (start 62.8402 65.941) (end 62.8452 65.936) (width 0.25) (layer "F.Cu") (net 9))
 (segment (start 63.5452 65.936) (end 64.4652 65.936) (width 0.25) (layer "F.Cu") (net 9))
 (segment (start 61.6202 65.941) (end 60.4038 65.941) (width 0.25) (layer "F.Cu") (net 9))
 (segment (start 65.6082 68.5546) (end 65.1502 68.0966) (width 0.25) (layer "F.Cu") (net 9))
 (segment (start 58.55 65.1) (end 58.55 65.5858) (width 0.25) (layer "F.Cu") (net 9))
 (segment (start 62.8452 65.936) (end 63.5452 65.936) (width 0.25) (layer "F.Cu") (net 9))
 (segment (start 61.727 52.847) (end 62.1942 52.847) (width 0.25) (layer "F.Cu") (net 9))
 (segment (start 68.5546 68.5292) (end 65.6336 68.5292) (width 0.25) (layer "F.Cu") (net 9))
 (segment (start 65.1502 66.711) (end 65.1502 67.481) (width 0.25) (layer "F.Cu") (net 9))
 (segment (start 68.4754 54.6354) (end 68.83 54.99) (width 0.25) (layer "F.Cu") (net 9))
 (segment (start 63.627 53.497) (end 64.1396 53.497) (width 0.25) (layer "F.Cu") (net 9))
 (segment (start 65.278 54.6354) (end 68.4754 54.6354) (width 0.25) (layer "F.Cu") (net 9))
 (segment (start 62.1942 52.847) (end 62.8442 53.497) (width 0.25) (layer "F.Cu") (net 9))
 (segment (start 64.5202 66.081) (end 65.1502 66.711) (width 0.25) (layer "F.Cu") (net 9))
 (segment (start 61.6202 65.941) (end 62.8402 65.941) (width 0.25) (layer "F.Cu") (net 9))
 (segment (start 59.5628 65.1) (end 58.55 65.1) (width 0.25) (layer "F.Cu") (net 9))
 (segment (start 65.6336 68.5292) (end 65.6082 68.5546) (width 0.25) (layer "F.Cu") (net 9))
 (segment (start 63.627 53.497) (end 63.627 54.4068) (width 0.25) (layer "F.Cu") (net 9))
 (segment (start 64.1396 53.497) (end 65.278 54.6354) (width 0.25) (layer "F.Cu") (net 9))
 (segment (start 69.9008 67.183) (end 68.5546 68.5292) (width 0.25) (layer "F.Cu") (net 9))
 (segment (start 60.4038 65.941) (end 59.5628 65.1) (width 0.25) (layer "F.Cu") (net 9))
 (segment (start 69.9008 63.881) (end 69.9008 67.183) (width 0.25) (layer "F.Cu") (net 9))
 (segment (start 62.8442 53.497) (end 63.627 53.497) (width 0.25) (layer "F.Cu") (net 9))
 (segment (start 65.1502 68.0966) (end 65.1502 67.481) (width 0.25) (layer "F.Cu") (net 9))
 (segment (start 64.4652 65.936) (end 64.5202 65.881) (width 0.25) (layer "F.Cu") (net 9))
 (via (at 69.9008 63.881) (size 0.6) (drill 0.3) (layers "F.Cu" "B.Cu") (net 9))
 (via (at 68.83 54.99) (size 0.6) (drill 0.3) (layers "F.Cu" "B.Cu") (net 9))
 (segment (start 69.9008 56.0832) (end 68.83 55.0124) (width 0.25) (layer "B.Cu") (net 9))
 (segment (start 68.83 55.0124) (end 68.83 54.99) (width 0.25) (layer "B.Cu") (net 9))
 (segment (start 69.9008 63.881) (end 69.9008 56.0832) (width 0.25) (layer "B.Cu") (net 9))
 (segment (start 68.426 63.981) (end 68.4276 63.9826) (width 0.25) (layer "F.Cu") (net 1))
 (segment (start 66.7952 63.981) (end 66.7952 62.8252) (width 0.25) (layer "F.Cu") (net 1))
 (segment (start 66.7952 62.8252) (end 62.7 58.73) (width 0.25) (layer "F.Cu") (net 1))
 (segment (start 62.7 58.73) (end 63.02 58.73) (width 0.25) (layer "F.Cu") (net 1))
 (segment (start 66.7952 63.981) (end 68.426 63.981) (width 0.25) (layer "F.Cu") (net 1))
 (segment (start 57.6 62.56) (end 58.89 61.27) (width 0.25) (layer "F.Cu") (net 2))
 (segment (start 57.6 63.225) (end 57.6 62.56) (width 0.25) (layer "F.Cu") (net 2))
 (segment (start 58.89 61.27) (end 62.7 61.27) (width 0.25) (layer "F.Cu") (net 2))
 (segment (start 62.0058 63.225) (end 59.5 63.225) (width 0.25) (layer "F.Cu") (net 8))
 (segment (start 59.545 63.18) (end 59.5 63.225) (width 0.25) (layer "F.Cu") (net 8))
 (segment (start 64.5202 63.981) (end 62.7618 63.981) (width 0.25) (layer "F.Cu") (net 8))
 (segment (start 62.7618 63.981) (end 62.0058 63.225) (width 0.25) (layer "F.Cu") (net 8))
 (segment (start 66.7952 67.346) (end 66.6602 67.481) (width 0.25) (layer "F.Cu") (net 7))
 (segment (start 67.7164 67.3608) (end 68.4276 67.3608) (width 0.25) (layer "F.Cu") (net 7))
 (segment (start 66.7952 65.881) (end 66.7952 67.196) (width 0.25) (layer "F.Cu") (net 7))
 (segment (start 66.5226 67.481) (end 67.5962 67.481) (width 0.25) (layer "F.Cu") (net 7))
 (segment (start 66.5226 67.481) (end 66.1702 67.481) (width 0.25) (layer "F.Cu") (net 7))
 (segment (start 66.7952 67.196) (end 66.7952 67.346) (width 0.25) (layer "F.Cu") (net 7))
 (segment (start 66.6602 67.481) (end 66.5226 67.481) (width 0.25) (layer "F.Cu") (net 7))
 (segment (start 67.5962 67.481) (end 67.7164 67.3608) (width 0.25) (layer "F.Cu") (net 7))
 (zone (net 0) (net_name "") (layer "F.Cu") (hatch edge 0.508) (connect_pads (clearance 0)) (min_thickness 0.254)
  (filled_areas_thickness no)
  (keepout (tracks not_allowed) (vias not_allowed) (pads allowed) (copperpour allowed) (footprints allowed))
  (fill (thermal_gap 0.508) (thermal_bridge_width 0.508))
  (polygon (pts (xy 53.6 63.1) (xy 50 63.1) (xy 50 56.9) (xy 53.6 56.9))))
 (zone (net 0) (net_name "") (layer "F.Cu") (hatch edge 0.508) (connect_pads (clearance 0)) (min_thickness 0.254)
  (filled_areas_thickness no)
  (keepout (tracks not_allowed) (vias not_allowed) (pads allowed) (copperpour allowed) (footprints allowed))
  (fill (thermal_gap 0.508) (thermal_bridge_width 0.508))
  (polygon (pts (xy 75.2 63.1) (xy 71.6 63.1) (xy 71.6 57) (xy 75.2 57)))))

